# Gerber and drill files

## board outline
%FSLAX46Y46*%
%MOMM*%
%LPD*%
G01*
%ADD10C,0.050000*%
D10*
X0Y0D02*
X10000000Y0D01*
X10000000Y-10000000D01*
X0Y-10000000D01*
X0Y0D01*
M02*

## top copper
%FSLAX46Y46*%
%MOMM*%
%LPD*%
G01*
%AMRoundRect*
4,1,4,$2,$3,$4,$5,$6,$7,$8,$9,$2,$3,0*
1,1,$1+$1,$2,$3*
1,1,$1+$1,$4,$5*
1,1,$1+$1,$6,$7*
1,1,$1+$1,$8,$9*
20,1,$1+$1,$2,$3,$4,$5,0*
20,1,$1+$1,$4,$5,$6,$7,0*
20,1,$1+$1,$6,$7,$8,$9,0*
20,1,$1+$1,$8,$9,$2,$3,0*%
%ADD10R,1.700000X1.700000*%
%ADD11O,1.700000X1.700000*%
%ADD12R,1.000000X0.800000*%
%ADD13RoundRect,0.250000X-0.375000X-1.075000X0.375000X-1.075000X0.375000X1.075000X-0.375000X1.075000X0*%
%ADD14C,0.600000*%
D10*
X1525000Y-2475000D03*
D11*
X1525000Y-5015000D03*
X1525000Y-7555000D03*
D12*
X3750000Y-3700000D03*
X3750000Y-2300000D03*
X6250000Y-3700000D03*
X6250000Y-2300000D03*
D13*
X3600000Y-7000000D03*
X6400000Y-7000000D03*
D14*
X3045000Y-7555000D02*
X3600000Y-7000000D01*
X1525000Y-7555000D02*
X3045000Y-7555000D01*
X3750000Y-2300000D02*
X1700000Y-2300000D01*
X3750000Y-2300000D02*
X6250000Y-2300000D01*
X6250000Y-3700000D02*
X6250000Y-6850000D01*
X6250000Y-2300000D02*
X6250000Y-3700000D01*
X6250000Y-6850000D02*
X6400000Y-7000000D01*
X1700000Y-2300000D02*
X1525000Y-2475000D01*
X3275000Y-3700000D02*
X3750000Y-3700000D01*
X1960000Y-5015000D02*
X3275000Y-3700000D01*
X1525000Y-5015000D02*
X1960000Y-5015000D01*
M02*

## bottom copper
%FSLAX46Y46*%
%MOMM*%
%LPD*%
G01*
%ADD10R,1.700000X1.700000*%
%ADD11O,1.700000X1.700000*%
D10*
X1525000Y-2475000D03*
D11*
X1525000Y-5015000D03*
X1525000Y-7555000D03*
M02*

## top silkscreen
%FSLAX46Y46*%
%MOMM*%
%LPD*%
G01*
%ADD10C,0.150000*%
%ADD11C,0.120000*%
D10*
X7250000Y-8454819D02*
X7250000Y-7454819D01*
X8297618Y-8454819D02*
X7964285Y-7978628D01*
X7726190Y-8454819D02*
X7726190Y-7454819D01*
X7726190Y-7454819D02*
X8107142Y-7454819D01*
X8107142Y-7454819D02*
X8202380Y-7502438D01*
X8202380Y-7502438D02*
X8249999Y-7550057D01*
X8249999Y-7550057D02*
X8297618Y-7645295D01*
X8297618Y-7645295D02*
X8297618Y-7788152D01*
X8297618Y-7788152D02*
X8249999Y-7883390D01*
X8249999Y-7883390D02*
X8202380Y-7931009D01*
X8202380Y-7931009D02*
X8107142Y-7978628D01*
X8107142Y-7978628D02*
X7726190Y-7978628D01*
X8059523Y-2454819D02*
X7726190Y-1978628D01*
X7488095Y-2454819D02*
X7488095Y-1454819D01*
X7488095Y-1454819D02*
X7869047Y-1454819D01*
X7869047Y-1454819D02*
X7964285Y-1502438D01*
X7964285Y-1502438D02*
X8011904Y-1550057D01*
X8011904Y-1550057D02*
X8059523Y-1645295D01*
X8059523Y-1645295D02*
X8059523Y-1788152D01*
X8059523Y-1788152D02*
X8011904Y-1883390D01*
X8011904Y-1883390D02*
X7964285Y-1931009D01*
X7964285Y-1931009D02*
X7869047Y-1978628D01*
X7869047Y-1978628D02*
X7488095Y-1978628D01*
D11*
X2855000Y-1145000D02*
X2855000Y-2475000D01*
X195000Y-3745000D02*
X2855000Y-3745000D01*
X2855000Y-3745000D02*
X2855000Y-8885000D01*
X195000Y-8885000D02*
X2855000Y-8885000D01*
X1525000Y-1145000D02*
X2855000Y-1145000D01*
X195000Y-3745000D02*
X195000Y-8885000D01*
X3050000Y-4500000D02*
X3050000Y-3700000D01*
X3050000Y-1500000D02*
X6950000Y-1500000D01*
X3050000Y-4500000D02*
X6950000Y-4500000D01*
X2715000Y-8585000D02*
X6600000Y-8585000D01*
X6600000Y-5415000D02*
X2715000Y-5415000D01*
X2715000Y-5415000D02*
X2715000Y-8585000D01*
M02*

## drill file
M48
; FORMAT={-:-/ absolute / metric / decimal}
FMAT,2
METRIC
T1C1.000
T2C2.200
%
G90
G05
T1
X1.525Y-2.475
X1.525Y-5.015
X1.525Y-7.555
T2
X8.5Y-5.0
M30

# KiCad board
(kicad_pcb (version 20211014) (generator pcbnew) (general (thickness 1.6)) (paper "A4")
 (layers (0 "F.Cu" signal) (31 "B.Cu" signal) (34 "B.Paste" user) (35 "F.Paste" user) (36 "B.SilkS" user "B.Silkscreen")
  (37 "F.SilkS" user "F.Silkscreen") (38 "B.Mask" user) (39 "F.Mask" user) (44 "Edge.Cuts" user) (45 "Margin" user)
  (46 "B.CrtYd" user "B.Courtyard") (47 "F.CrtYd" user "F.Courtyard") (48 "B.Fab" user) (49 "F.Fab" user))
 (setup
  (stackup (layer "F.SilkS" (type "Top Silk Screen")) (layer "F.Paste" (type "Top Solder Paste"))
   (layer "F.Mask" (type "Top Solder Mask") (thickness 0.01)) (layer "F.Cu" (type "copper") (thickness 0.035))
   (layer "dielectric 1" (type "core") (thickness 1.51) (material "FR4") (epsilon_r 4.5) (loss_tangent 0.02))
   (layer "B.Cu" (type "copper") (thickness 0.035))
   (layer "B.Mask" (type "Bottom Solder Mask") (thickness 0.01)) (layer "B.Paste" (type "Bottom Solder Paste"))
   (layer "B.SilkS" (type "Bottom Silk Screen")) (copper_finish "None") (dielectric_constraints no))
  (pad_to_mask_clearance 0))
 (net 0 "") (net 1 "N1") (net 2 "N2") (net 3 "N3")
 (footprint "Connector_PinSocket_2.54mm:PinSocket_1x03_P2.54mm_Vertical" (layer "F.Cu") (at 1.525 2.475)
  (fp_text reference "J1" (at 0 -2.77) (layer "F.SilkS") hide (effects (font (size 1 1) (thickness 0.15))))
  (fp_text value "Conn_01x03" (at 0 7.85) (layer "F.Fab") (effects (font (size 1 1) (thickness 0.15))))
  (fp_line (start 1.33 -1.33) (end 1.33 0) (layer "F.SilkS") (width 0.12))
  (fp_line (start -1.33 1.27) (end 1.33 1.27) (layer "F.SilkS") (width 0.12))
  (fp_line (start 1.33 1.27) (end 1.33 6.41) (layer "F.SilkS") (width 0.12))
  (fp_line (start -1.33 6.41) (end 1.33 6.41) (layer "F.SilkS") (width 0.12))
  (fp_line (start 0 -1.33) (end 1.33 -1.33) (layer "F.SilkS") (width 0.12))
  (fp_line (start -1.33 1.27) (end -1.33 6.41) (layer "F.SilkS") (width 0.12))
  (pad "1" thru_hole rect locked (at 0 0) (size 1.7 1.7) (drill 1) (layers *.Cu *.Mask) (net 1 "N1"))
  (pad "2" thru_hole oval locked (at 0 2.54) (size 1.7 1.7) (drill 1) (layers *.Cu *.Mask) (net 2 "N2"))
  (pad "3" thru_hole oval locked (at 0 5.08) (size 1.7 1.7) (drill 1) (layers *.Cu *.Mask) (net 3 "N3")))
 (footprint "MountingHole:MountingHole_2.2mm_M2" (layer "F.Cu") (at 8.5 5)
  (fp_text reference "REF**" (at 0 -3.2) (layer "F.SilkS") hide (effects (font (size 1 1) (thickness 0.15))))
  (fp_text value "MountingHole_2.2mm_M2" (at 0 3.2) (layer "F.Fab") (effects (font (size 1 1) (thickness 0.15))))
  (pad "" np_thru_hole circle locked (at 0 0) (size 2.2 2.2) (drill 2.2) (layers *.Cu *.Mask)))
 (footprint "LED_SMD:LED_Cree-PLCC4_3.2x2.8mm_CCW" (layer "F.Cu") (at 5 3)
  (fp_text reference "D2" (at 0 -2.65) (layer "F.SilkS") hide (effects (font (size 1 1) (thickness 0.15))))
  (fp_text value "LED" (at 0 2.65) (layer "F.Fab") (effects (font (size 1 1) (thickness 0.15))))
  (fp_line (start -1.95 1.5) (end -1.95 0.7) (layer "F.SilkS") (width 0.12))
  (fp_line (start -1.95 -1.5) (end 1.95 -1.5) (layer "F.SilkS") (width 0.12))
  (fp_line (start -1.95 1.5) (end 1.95 1.5) (layer "F.SilkS") (width 0.12))
  (pad "1" smd rect (at -1.25 0.7) (size 1 0.8) (layers "F.Cu" "F.Paste" "F.Mask") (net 2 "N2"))
  (pad "2" smd rect (at -1.25 -0.7) (size 1 0.8) (layers "F.Cu" "F.Paste" "F.Mask") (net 1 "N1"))
  (pad "2" smd rect (at 1.25 0.7) (size 1 0.8) (layers "F.Cu" "F.Paste" "F.Mask") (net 1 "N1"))
  (pad "2" smd rect (at 1.25 -0.7) (size 1 0.8) (layers "F.Cu" "F.Paste" "F.Mask") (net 1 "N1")))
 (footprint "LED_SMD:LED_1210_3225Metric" (layer "F.Cu") (at 5 7)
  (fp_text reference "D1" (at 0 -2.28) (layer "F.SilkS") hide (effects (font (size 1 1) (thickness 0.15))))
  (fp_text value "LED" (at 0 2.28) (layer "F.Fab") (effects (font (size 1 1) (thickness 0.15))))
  (fp_line (start -2.285 1.585) (end 1.6 1.585) (layer "F.SilkS") (width 0.12))
  (fp_line (start 1.6 -1.585) (end -2.285 -1.585) (layer "F.SilkS") (width 0.12))
  (fp_line (start -2.285 -1.585) (end -2.285 1.585) (layer "F.SilkS") (width 0.12))
  (pad "1" smd roundrect (at -1.4 0) (size 1.25 2.65) (layers "F.Cu" "F.Paste" "F.Mask") (roundrect_rratio 0.2) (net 3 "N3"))
  (pad "2" smd roundrect (at 1.4 0) (size 1.25 2.65) (layers "F.Cu" "F.Paste" "F.Mask") (roundrect_rratio 0.2) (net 1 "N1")))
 (gr_rect (start 0 0) (end 10 10) (layer "Edge.Cuts") (width 0.05) (fill none))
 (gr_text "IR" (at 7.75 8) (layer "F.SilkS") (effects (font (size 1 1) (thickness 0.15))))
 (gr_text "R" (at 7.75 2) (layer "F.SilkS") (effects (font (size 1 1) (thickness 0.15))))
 (segment (start 3.045 7.555) (end 3.6 7) (width 0.6) (layer "F.Cu") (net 3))
 (segment (start 1.525 7.555) (end 3.045 7.555) (width 0.6) (layer "F.Cu") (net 3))
 (segment (start 3.75 2.3) (end 1.7 2.3) (width 0.6) (layer "F.Cu") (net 1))
 (segment (start 3.75 2.3) (end 6.25 2.3) (width 0.6) (layer "F.Cu") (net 1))
 (segment (start 6.25 3.7) (end 6.25 6.85) (width 0.6) (layer "F.Cu") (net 1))
 (segment (start 6.25 2.3) (end 6.25 3.7) (width 0.6) (layer "F.Cu") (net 1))
 (segment (start 6.25 6.85) (end 6.4 7) (width 0.6) (layer "F.Cu") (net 1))
 (segment (start 1.7 2.3) (end 1.525 2.475) (width 0.6) (layer "F.Cu") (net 1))
 (segment (start 3.275 3.7) (end 3.75 3.7) (width 0.6) (layer "F.Cu") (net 2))
 (segment (start 1.96 5.015) (end 3.275 3.7) (width 0.6) (layer "F.Cu") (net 2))
 (segment (start 1.525 5.015) (end 1.96 5.015) (width 0.6) (layer "F.Cu") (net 2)))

